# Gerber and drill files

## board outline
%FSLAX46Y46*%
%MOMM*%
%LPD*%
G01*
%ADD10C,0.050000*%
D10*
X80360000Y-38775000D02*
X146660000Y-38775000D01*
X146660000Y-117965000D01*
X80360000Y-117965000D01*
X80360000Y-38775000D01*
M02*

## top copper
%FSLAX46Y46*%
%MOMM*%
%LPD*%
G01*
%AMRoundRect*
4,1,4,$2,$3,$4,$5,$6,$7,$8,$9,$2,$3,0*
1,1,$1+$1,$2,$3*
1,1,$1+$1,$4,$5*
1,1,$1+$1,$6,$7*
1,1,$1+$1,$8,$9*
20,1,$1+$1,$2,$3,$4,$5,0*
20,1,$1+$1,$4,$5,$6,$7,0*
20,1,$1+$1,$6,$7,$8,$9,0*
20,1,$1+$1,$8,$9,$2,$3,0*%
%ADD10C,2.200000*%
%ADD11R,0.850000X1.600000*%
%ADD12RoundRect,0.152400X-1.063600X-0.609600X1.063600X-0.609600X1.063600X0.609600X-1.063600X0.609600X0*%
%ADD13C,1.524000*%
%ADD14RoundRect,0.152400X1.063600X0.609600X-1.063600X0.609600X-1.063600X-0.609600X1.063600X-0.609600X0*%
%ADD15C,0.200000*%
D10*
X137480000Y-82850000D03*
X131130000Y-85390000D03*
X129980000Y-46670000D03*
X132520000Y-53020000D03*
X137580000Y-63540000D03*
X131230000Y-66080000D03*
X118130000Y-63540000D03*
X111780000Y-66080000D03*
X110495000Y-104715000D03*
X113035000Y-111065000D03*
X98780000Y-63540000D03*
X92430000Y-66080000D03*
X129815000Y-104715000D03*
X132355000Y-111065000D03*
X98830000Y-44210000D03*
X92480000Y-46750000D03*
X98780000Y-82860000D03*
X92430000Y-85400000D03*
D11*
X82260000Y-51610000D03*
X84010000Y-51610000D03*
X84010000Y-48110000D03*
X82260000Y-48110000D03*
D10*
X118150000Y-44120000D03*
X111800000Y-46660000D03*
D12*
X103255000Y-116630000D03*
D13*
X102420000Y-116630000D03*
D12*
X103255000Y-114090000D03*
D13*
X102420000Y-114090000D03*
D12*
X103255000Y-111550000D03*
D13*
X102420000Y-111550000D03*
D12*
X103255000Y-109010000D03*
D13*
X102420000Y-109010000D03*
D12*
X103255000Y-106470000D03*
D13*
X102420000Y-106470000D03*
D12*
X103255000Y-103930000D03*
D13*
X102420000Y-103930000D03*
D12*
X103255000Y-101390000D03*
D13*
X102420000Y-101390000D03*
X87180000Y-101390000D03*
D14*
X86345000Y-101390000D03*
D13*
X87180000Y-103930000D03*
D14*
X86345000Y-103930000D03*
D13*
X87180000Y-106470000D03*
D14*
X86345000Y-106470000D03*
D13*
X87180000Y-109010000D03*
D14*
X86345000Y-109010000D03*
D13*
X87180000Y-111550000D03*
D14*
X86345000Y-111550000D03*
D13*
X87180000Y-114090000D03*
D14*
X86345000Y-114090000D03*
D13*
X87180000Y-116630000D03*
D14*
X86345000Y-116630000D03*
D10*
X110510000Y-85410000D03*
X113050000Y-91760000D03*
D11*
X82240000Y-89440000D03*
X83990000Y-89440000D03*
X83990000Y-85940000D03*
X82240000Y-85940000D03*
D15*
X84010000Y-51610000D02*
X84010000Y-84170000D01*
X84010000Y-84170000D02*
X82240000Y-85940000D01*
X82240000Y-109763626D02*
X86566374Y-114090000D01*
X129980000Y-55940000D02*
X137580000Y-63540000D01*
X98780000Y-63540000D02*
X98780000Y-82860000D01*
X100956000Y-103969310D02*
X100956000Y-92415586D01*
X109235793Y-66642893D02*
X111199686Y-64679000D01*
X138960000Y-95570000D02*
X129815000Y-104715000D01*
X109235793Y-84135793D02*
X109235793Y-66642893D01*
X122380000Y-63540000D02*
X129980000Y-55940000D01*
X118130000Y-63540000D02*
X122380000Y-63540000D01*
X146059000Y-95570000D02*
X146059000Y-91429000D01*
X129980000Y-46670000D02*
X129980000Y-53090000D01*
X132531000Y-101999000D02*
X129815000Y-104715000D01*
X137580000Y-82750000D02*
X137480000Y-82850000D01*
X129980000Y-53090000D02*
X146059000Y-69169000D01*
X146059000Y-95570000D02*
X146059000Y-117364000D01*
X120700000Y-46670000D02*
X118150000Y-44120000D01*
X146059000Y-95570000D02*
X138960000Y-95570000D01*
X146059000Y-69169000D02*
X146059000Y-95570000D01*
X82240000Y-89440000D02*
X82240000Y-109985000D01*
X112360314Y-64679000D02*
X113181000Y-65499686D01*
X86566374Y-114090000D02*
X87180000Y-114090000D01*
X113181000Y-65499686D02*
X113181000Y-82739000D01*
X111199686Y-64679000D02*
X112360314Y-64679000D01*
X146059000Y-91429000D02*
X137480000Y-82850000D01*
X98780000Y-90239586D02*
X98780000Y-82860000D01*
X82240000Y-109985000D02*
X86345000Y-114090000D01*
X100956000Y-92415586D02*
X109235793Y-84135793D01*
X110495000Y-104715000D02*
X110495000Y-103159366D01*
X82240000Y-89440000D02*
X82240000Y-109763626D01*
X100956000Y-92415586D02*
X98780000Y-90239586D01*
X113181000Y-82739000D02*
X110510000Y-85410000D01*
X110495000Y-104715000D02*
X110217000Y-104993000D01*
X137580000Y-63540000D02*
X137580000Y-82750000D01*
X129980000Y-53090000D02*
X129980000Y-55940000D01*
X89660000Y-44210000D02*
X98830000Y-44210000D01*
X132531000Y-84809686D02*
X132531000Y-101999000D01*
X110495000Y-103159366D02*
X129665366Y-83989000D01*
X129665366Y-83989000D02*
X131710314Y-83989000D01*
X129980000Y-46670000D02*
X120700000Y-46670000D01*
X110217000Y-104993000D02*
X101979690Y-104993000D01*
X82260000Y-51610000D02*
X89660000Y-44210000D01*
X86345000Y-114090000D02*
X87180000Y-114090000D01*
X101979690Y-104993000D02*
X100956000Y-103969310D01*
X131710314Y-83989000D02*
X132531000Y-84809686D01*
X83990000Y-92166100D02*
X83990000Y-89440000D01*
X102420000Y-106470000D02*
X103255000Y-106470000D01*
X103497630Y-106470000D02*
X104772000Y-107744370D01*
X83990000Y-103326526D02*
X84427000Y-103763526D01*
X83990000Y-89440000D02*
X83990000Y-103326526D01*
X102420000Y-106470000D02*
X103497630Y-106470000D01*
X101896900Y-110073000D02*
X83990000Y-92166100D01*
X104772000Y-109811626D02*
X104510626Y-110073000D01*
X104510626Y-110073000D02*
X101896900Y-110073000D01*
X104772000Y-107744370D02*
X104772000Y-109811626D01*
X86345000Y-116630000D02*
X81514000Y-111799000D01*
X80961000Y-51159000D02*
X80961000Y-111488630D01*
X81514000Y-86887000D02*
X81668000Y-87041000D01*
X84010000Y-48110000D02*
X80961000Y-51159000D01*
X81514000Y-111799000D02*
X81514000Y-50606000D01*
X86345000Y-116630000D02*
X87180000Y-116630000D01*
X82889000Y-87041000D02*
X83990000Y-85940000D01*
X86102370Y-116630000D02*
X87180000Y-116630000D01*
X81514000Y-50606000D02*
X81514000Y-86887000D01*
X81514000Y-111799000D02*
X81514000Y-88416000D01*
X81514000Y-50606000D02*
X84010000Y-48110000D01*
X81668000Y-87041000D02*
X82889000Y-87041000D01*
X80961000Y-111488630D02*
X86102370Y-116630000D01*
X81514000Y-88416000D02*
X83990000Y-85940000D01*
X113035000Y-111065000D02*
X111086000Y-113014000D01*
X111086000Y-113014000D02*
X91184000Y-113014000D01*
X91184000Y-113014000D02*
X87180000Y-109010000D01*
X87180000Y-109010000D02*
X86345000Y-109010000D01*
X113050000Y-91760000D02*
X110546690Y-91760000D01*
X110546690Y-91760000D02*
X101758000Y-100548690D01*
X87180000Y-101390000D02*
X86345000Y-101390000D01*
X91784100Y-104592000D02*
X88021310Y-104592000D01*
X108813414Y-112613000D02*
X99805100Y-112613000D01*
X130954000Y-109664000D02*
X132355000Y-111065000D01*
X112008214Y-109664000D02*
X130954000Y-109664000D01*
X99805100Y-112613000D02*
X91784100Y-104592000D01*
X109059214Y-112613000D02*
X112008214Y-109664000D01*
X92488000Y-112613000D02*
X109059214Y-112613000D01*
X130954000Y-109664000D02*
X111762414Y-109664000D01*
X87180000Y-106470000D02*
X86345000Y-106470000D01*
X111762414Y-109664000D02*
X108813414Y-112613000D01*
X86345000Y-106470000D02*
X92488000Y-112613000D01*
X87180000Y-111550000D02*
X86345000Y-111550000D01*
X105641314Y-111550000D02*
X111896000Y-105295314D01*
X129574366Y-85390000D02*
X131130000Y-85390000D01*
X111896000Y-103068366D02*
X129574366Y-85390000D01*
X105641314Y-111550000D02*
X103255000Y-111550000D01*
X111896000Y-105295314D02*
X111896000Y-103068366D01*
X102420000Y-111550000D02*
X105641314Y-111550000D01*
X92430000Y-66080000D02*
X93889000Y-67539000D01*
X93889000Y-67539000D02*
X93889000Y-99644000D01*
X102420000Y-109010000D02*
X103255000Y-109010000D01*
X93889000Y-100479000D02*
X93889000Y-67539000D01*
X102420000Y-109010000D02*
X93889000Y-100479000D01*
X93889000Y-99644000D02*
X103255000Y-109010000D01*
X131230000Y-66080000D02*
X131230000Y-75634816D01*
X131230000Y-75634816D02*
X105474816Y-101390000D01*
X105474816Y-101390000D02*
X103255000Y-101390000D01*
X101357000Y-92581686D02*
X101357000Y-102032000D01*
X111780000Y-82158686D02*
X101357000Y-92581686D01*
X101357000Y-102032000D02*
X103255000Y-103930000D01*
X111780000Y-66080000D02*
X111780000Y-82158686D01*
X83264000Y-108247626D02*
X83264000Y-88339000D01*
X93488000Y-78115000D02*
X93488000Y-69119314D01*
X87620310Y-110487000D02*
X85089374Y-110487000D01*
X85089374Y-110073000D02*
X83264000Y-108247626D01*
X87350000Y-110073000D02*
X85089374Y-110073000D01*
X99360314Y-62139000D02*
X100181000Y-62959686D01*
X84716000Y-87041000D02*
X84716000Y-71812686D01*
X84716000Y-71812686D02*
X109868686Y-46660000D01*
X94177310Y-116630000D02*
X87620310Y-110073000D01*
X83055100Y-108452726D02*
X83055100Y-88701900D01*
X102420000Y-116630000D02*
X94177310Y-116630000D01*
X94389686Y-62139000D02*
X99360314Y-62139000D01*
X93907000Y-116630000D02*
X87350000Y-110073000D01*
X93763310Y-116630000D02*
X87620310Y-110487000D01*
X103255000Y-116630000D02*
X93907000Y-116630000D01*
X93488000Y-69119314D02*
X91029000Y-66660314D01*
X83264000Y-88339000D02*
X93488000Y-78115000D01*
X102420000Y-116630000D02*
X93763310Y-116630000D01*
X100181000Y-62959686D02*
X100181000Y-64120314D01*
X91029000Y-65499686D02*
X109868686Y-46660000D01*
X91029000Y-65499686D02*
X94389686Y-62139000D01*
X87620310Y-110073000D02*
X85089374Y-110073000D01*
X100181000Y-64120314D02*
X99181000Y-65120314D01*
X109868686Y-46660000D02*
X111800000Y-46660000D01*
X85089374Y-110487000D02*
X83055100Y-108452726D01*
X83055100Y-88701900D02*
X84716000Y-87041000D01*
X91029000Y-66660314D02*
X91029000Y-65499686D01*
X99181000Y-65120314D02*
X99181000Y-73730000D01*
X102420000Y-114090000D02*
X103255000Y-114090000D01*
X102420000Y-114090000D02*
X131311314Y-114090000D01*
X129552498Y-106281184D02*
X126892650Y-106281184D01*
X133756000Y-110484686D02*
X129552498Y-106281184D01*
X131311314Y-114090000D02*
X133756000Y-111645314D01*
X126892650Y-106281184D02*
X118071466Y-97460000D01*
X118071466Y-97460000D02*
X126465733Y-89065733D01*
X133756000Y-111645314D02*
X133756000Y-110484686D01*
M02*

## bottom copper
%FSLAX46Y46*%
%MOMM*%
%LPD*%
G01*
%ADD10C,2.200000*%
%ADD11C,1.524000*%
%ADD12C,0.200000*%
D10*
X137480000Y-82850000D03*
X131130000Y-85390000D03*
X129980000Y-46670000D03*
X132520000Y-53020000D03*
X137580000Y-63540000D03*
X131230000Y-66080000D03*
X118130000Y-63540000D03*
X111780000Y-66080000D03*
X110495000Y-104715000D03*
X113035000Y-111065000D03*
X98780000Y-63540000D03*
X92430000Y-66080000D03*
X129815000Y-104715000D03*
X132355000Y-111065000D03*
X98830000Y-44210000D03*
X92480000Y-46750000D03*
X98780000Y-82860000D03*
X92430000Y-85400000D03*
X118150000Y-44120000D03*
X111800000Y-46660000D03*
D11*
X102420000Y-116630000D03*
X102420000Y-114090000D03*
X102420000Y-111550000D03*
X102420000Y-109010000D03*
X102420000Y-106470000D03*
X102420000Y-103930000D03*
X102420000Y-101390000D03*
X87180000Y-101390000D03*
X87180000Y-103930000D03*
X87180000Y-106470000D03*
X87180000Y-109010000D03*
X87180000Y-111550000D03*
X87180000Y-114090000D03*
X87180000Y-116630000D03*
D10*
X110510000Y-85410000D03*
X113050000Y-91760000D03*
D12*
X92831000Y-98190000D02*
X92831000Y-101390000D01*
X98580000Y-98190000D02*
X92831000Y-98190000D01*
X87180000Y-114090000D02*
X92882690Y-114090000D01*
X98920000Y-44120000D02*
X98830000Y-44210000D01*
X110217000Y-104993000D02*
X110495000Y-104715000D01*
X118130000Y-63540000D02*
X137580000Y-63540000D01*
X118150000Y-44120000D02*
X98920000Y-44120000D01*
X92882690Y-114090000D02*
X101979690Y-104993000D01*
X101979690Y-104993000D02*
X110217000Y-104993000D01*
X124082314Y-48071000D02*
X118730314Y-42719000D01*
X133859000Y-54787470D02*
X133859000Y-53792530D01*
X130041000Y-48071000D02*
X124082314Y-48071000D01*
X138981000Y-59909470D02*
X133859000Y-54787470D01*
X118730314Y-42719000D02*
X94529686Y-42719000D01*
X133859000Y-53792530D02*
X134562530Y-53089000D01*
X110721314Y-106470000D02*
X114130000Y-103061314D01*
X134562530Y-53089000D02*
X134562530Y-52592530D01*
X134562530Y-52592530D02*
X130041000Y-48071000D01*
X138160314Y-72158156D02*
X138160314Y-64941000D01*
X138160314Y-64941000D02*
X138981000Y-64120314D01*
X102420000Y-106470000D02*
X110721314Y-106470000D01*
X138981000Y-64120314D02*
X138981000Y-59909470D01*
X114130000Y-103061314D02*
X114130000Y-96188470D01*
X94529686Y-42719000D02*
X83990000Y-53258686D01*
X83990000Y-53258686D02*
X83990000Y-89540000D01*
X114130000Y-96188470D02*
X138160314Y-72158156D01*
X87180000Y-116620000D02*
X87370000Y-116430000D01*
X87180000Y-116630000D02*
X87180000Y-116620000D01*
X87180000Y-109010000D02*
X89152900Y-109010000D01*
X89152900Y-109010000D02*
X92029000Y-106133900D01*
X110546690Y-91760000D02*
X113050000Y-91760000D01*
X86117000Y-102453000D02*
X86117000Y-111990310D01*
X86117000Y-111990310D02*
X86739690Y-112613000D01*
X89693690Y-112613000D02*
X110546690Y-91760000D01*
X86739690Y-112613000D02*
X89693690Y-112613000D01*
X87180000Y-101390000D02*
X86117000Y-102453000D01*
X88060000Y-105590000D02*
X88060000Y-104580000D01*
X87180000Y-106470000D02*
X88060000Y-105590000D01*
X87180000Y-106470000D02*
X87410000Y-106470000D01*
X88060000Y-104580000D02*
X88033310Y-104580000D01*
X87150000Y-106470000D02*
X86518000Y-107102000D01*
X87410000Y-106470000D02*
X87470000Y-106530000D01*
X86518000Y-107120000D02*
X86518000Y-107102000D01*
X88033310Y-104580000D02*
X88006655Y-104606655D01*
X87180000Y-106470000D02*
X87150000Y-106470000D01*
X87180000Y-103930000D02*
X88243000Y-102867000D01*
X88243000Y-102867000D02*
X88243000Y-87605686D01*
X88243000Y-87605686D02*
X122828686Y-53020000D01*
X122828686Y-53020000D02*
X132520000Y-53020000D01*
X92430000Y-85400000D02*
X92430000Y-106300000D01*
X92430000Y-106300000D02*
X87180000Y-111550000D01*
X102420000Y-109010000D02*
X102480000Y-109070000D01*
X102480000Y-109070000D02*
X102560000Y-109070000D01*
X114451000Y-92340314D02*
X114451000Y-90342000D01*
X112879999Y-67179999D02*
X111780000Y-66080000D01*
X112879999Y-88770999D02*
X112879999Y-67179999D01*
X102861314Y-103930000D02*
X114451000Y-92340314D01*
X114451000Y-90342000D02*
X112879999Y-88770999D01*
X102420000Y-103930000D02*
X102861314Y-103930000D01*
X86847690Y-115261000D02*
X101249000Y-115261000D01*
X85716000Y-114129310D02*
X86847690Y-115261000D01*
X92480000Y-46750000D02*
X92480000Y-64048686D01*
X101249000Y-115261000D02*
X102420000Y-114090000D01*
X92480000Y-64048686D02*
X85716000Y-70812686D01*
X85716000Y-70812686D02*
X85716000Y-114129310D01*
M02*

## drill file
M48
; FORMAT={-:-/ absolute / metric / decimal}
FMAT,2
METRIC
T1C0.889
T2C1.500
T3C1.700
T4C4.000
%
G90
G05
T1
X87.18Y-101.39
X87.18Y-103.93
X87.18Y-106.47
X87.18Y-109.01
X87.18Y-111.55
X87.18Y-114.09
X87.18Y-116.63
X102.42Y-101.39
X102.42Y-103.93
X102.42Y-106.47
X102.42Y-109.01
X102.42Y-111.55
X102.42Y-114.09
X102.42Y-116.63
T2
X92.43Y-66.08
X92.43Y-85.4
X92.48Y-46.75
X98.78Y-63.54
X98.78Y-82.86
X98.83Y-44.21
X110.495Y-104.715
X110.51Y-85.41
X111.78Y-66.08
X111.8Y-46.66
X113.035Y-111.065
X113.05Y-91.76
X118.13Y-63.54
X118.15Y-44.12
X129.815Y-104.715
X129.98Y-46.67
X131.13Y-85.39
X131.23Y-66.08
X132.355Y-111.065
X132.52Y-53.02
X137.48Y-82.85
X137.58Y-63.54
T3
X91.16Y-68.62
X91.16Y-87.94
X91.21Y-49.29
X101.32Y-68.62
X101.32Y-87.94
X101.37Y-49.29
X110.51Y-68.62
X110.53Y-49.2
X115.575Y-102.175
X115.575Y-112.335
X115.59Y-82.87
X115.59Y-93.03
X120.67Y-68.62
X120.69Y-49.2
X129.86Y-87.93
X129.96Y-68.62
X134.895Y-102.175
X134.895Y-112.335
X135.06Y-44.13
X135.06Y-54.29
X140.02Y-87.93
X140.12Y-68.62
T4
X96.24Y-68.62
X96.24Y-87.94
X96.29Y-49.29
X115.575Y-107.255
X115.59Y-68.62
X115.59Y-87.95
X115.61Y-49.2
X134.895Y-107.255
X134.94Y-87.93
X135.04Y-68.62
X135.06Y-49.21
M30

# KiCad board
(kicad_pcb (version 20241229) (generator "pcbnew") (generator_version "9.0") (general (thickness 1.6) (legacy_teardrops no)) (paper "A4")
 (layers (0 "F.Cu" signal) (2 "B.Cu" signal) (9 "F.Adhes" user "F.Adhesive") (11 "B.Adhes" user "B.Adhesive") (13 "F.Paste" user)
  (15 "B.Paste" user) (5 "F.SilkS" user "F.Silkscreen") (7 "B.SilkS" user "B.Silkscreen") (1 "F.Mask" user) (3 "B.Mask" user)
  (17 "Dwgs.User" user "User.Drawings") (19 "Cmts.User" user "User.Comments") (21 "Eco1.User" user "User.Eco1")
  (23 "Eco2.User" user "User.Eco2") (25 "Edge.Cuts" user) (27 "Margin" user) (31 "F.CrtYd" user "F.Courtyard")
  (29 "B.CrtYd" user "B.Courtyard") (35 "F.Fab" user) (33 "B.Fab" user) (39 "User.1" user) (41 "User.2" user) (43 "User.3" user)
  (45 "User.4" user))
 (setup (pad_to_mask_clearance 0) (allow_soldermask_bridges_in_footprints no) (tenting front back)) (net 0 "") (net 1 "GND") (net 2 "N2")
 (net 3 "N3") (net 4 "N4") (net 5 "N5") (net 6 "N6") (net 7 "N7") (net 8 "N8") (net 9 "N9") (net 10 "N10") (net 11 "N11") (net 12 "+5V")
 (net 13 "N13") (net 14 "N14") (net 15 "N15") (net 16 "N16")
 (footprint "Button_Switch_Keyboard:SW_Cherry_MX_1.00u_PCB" (layer "F.Cu") (at 137.48 82.85)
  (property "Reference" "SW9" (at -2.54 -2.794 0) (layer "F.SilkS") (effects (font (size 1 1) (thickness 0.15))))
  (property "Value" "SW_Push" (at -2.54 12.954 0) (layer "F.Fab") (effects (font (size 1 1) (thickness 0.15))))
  (pad "" np_thru_hole circle (at -7.62 5.08) (size 1.7 1.7) (drill 1.7) (layers "*.Cu" "*.Mask"))
  (pad "" np_thru_hole circle (at -2.54 5.08) (size 4 4) (drill 4) (layers "*.Cu" "*.Mask"))
  (pad "" np_thru_hole circle (at 2.54 5.08) (size 1.7 1.7) (drill 1.7) (layers "*.Cu" "*.Mask"))
  (pad "1" thru_hole circle (at 0 0) (size 2.2 2.2) (drill 1.5) (layers "*.Cu" "*.Mask") (remove_unused_layers no) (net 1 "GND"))
  (pad "2" thru_hole circle (at -6.35 2.54) (size 2.2 2.2) (drill 1.5) (layers "*.Cu" "*.Mask") (remove_unused_layers no) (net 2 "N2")))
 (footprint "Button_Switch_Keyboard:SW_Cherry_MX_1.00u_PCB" (layer "F.Cu") (at 129.98 46.67 90)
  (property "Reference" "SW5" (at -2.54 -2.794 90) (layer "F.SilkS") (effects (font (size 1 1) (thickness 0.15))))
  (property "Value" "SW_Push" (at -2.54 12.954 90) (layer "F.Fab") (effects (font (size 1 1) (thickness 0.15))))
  (pad "" np_thru_hole circle (at -7.62 5.08 90) (size 1.7 1.7) (drill 1.7) (layers "*.Cu" "*.Mask"))
  (pad "" np_thru_hole circle (at -2.54 5.08 90) (size 4 4) (drill 4) (layers "*.Cu" "*.Mask"))
  (pad "" np_thru_hole circle (at 2.54 5.08 90) (size 1.7 1.7) (drill 1.7) (layers "*.Cu" "*.Mask"))
  (pad "1" thru_hole circle (at 0 0 90) (size 2.2 2.2) (drill 1.5) (layers "*.Cu" "*.Mask") (remove_unused_layers no) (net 1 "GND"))
  (pad "2" thru_hole circle (at -6.35 2.54 90) (size 2.2 2.2) (drill 1.5) (layers "*.Cu" "*.Mask") (remove_unused_layers no) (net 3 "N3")))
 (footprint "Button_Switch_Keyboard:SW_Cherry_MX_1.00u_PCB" (layer "F.Cu") (at 137.58 63.54)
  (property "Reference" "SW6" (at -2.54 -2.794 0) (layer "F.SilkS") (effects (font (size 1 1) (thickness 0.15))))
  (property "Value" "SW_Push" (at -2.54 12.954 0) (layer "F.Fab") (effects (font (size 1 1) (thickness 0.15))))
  (pad "" np_thru_hole circle (at -7.62 5.08) (size 1.7 1.7) (drill 1.7) (layers "*.Cu" "*.Mask"))
  (pad "" np_thru_hole circle (at -2.54 5.08) (size 4 4) (drill 4) (layers "*.Cu" "*.Mask"))
  (pad "" np_thru_hole circle (at 2.54 5.08) (size 1.7 1.7) (drill 1.7) (layers "*.Cu" "*.Mask"))
  (pad "1" thru_hole circle (at 0 0) (size 2.2 2.2) (drill 1.5) (layers "*.Cu" "*.Mask") (remove_unused_layers no) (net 1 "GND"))
  (pad "2" thru_hole circle (at -6.35 2.54) (size 2.2 2.2) (drill 1.5) (layers "*.Cu" "*.Mask") (remove_unused_layers no) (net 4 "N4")))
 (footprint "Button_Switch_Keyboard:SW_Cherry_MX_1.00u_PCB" (layer "F.Cu") (at 118.13 63.54)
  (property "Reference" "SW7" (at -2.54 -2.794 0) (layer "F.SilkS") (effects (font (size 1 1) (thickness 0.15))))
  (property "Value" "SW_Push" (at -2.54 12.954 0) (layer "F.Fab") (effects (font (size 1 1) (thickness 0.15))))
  (pad "" np_thru_hole circle (at -7.62 5.08) (size 1.7 1.7) (drill 1.7) (layers "*.Cu" "*.Mask"))
  (pad "" np_thru_hole circle (at -2.54 5.08) (size 4 4) (drill 4) (layers "*.Cu" "*.Mask"))
  (pad "" np_thru_hole circle (at 2.54 5.08) (size 1.7 1.7) (drill 1.7) (layers "*.Cu" "*.Mask"))
  (pad "1" thru_hole circle (at 0 0) (size 2.2 2.2) (drill 1.5) (layers "*.Cu" "*.Mask") (remove_unused_layers no) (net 1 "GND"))
  (pad "2" thru_hole circle (at -6.35 2.54) (size 2.2 2.2) (drill 1.5) (layers "*.Cu" "*.Mask") (remove_unused_layers no) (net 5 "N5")))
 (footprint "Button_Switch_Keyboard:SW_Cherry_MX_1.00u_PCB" (layer "F.Cu") (at 110.495 104.715 90)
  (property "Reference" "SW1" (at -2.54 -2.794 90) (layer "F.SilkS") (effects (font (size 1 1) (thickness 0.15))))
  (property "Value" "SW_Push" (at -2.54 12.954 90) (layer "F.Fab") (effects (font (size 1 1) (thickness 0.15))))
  (pad "" np_thru_hole circle (at -7.62 5.08 90) (size 1.7 1.7) (drill 1.7) (layers "*.Cu" "*.Mask"))
  (pad "" np_thru_hole circle (at -2.54 5.08 90) (size 4 4) (drill 4) (layers "*.Cu" "*.Mask"))
  (pad "" np_thru_hole circle (at 2.54 5.08 90) (size 1.7 1.7) (drill 1.7) (layers "*.Cu" "*.Mask"))
  (pad "1" thru_hole circle (at 0 0 90) (size 2.2 2.2) (drill 1.5) (layers "*.Cu" "*.Mask") (remove_unused_layers no) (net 1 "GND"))
  (pad "2" thru_hole circle (at -6.35 2.54 90) (size 2.2 2.2) (drill 1.5) (layers "*.Cu" "*.Mask") (remove_unused_layers no) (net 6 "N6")))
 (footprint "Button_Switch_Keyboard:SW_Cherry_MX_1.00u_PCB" (layer "F.Cu") (at 98.78 63.54)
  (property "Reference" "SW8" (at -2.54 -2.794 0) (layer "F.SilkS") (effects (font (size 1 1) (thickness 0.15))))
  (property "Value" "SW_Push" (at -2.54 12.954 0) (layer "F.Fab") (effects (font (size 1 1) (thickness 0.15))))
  (pad "" np_thru_hole circle (at -7.62 5.08) (size 1.7 1.7) (drill 1.7) (layers "*.Cu" "*.Mask"))
  (pad "" np_thru_hole circle (at -2.54 5.08) (size 4 4) (drill 4) (layers "*.Cu" "*.Mask"))
  (pad "" np_thru_hole circle (at 2.54 5.08) (size 1.7 1.7) (drill 1.7) (layers "*.Cu" "*.Mask"))
  (pad "1" thru_hole circle (at 0 0) (size 2.2 2.2) (drill 1.5) (layers "*.Cu" "*.Mask") (remove_unused_layers no) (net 1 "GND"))
  (pad "2" thru_hole circle (at -6.35 2.54) (size 2.2 2.2) (drill 1.5) (layers "*.Cu" "*.Mask") (remove_unused_layers no) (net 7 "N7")))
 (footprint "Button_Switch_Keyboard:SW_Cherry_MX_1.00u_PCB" (layer "F.Cu") (at 129.815 104.715 90)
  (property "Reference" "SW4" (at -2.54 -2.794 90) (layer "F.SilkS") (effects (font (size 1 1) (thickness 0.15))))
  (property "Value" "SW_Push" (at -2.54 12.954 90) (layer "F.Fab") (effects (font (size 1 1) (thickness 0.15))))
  (pad "" np_thru_hole circle (at -7.62 5.08 90) (size 1.7 1.7) (drill 1.7) (layers "*.Cu" "*.Mask"))
  (pad "" np_thru_hole circle (at -2.54 5.08 90) (size 4 4) (drill 4) (layers "*.Cu" "*.Mask"))
  (pad "" np_thru_hole circle (at 2.54 5.08 90) (size 1.7 1.7) (drill 1.7) (layers "*.Cu" "*.Mask"))
  (pad "1" thru_hole circle (at 0 0 90) (size 2.2 2.2) (drill 1.5) (layers "*.Cu" "*.Mask") (remove_unused_layers no) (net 1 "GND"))
  (pad "2" thru_hole circle (at -6.35 2.54 90) (size 2.2 2.2) (drill 1.5) (layers "*.Cu" "*.Mask") (remove_unused_layers no) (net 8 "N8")))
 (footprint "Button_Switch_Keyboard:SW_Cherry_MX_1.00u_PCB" (layer "F.Cu") (at 98.83 44.21)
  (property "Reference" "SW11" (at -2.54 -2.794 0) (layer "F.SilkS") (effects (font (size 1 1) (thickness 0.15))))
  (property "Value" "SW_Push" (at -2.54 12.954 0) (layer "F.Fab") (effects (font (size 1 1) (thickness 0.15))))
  (pad "" np_thru_hole circle (at -7.62 5.08) (size 1.7 1.7) (drill 1.7) (layers "*.Cu" "*.Mask"))
  (pad "" np_thru_hole circle (at -2.54 5.08) (size 4 4) (drill 4) (layers "*.Cu" "*.Mask"))
  (pad "" np_thru_hole circle (at 2.54 5.08) (size 1.7 1.7) (drill 1.7) (layers "*.Cu" "*.Mask"))
  (pad "1" thru_hole circle (at 0 0) (size 2.2 2.2) (drill 1.5) (layers "*.Cu" "*.Mask") (remove_unused_layers no) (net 1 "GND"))
  (pad "2" thru_hole circle (at -6.35 2.54) (size 2.2 2.2) (drill 1.5) (layers "*.Cu" "*.Mask") (remove_unused_layers no) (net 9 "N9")))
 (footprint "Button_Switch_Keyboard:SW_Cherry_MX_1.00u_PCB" (layer "F.Cu") (at 98.78 82.86)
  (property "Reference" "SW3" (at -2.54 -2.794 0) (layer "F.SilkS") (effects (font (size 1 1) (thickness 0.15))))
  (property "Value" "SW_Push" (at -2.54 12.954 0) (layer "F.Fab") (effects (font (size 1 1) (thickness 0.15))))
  (pad "" np_thru_hole circle (at -7.62 5.08) (size 1.7 1.7) (drill 1.7) (layers "*.Cu" "*.Mask"))
  (pad "" np_thru_hole circle (at -2.54 5.08) (size 4 4) (drill 4) (layers "*.Cu" "*.Mask"))
  (pad "" np_thru_hole circle (at 2.54 5.08) (size 1.7 1.7) (drill 1.7) (layers "*.Cu" "*.Mask"))
  (pad "1" thru_hole circle (at 0 0) (size 2.2 2.2) (drill 1.5) (layers "*.Cu" "*.Mask") (remove_unused_layers no) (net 1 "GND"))
  (pad "2" thru_hole circle (at -6.35 2.54) (size 2.2 2.2) (drill 1.5) (layers "*.Cu" "*.Mask") (remove_unused_layers no) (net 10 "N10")))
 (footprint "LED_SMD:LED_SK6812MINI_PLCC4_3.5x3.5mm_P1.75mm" (layer "F.Cu") (at 83.135 49.86 90)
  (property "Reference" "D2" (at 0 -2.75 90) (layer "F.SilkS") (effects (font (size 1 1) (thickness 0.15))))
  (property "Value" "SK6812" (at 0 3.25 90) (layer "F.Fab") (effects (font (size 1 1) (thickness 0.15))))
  (pad "1" smd rect (at -1.75 -0.875 90) (size 1.6 0.85) (layers "F.Cu" "F.Mask" "F.Paste") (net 1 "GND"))
  (pad "2" smd rect (at -1.75 0.875 90) (size 1.6 0.85) (layers "F.Cu" "F.Mask" "F.Paste") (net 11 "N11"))
  (pad "3" smd rect (at 1.75 0.875 90) (size 1.6 0.85) (layers "F.Cu" "F.Mask" "F.Paste") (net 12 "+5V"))
  (pad "4" smd rect (at 1.75 -0.875 90) (size 1.6 0.85) (layers "F.Cu" "F.Mask" "F.Paste") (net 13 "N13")))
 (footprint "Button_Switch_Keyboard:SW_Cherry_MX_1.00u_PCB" (layer "F.Cu") (at 118.15 44.12)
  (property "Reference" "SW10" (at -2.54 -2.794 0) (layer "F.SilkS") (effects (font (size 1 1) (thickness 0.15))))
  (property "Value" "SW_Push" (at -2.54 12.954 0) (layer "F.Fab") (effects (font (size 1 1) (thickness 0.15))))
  (pad "" np_thru_hole circle (at -7.62 5.08) (size 1.7 1.7) (drill 1.7) (layers "*.Cu" "*.Mask"))
  (pad "" np_thru_hole circle (at -2.54 5.08) (size 4 4) (drill 4) (layers "*.Cu" "*.Mask"))
  (pad "" np_thru_hole circle (at 2.54 5.08) (size 1.7 1.7) (drill 1.7) (layers "*.Cu" "*.Mask"))
  (pad "1" thru_hole circle (at 0 0) (size 2.2 2.2) (drill 1.5) (layers "*.Cu" "*.Mask") (remove_unused_layers no) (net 1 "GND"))
  (pad "2" thru_hole circle (at -6.35 2.54) (size 2.2 2.2) (drill 1.5) (layers "*.Cu" "*.Mask") (remove_unused_layers no) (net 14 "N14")))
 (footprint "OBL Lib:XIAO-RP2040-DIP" (layer "F.Cu") (at 94.8 109.01 180)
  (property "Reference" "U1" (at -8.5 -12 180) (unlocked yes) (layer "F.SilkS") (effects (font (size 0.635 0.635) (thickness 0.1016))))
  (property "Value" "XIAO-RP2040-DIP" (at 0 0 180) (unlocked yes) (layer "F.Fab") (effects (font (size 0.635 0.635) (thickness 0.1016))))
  (pad "1" smd roundrect (at -8.455 -7.62) (size 2.432 1.524) (layers "F.Cu" "F.Mask") (roundrect_rratio 0.1) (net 14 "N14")
   (thermal_bridge_angle 45))
  (pad "1" thru_hole circle (at -7.62 -7.62) (size 1.524 1.524) (drill 0.889) (layers "*.Cu" "*.Mask") (remove_unused_layers no)
   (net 14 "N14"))
  (pad "2" smd roundrect (at -8.455 -5.08) (size 2.432 1.524) (layers "F.Cu" "F.Mask") (roundrect_rratio 0.1) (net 9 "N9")
   (thermal_bridge_angle 45))
  (pad "2" thru_hole circle (at -7.62 -5.08) (size 1.524 1.524) (drill 0.889) (layers "*.Cu" "*.Mask") (remove_unused_layers no)
   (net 9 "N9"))
  (pad "3" smd roundrect (at -8.455 -2.54) (size 2.432 1.524) (layers "F.Cu" "F.Mask") (roundrect_rratio 0.1) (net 2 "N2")
   (thermal_bridge_angle 45))
  (pad "3" thru_hole circle (at -7.62 -2.54) (size 1.524 1.524) (drill 0.889) (layers "*.Cu" "*.Mask") (remove_unused_layers no)
   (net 2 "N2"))
  (pad "4" smd roundrect (at -8.455 0) (size 2.432 1.524) (layers "F.Cu" "F.Mask") (roundrect_rratio 0.1) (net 7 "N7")
   (thermal_bridge_angle 45))
  (pad "4" thru_hole circle (at -7.62 0) (size 1.524 1.524) (drill 0.889) (layers "*.Cu" "*.Mask") (remove_unused_layers no) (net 7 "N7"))
  (pad "5" smd roundrect (at -8.455 2.54) (size 2.432 1.524) (layers "F.Cu" "F.Mask") (roundrect_rratio 0.1) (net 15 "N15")
   (thermal_bridge_angle 45))
  (pad "5" thru_hole circle (at -7.62 2.54) (size 1.524 1.524) (drill 0.889) (layers "*.Cu" "*.Mask") (remove_unused_layers no)
   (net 15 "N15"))
  (pad "6" smd roundrect (at -8.455 5.08) (size 2.432 1.524) (layers "F.Cu" "F.Mask") (roundrect_rratio 0.1) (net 5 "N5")
   (thermal_bridge_angle 45))
  (pad "6" thru_hole circle (at -7.62 5.08) (size 1.524 1.524) (drill 0.889) (layers "*.Cu" "*.Mask") (remove_unused_layers no) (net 5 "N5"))
  (pad "7" smd roundrect (at -8.455 7.62) (size 2.432 1.524) (layers "F.Cu" "F.Mask") (roundrect_rratio 0.1) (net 4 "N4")
   (thermal_bridge_angle 45))
  (pad "7" thru_hole circle (at -7.62 7.62) (size 1.524 1.524) (drill 0.889) (layers "*.Cu" "*.Mask") (remove_unused_layers no) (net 4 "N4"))
  (pad "8" thru_hole circle (at 7.62 7.62 180) (size 1.524 1.524) (drill 0.889) (layers "*.Cu" "*.Mask") (remove_unused_layers no)
   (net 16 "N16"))
  (pad "8" smd roundrect (at 8.455 7.62 180) (size 2.432 1.524) (layers "F.Cu" "F.Mask") (roundrect_rratio 0.1) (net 16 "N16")
   (thermal_bridge_angle 45))
  (pad "9" thru_hole circle (at 7.62 5.08 180) (size 1.524 1.524) (drill 0.889) (layers "*.Cu" "*.Mask") (remove_unused_layers no)
   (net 3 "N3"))
  (pad "9" smd roundrect (at 8.455 5.08 180) (size 2.432 1.524) (layers "F.Cu" "F.Mask") (roundrect_rratio 0.1) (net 3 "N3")
   (thermal_bridge_angle 45))
  (pad "10" thru_hole circle (at 7.62 2.54 180) (size 1.524 1.524) (drill 0.889) (layers "*.Cu" "*.Mask") (remove_unused_layers no)
   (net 8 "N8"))
  (pad "10" smd roundrect (at 8.455 2.54 180) (size 2.432 1.524) (layers "F.Cu" "F.Mask") (roundrect_rratio 0.1) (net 8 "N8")
   (thermal_bridge_angle 45))
  (pad "11" thru_hole circle (at 7.62 0 180) (size 1.524 1.524) (drill 0.889) (layers "*.Cu" "*.Mask") (remove_unused_layers no)
   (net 6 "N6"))
  (pad "11" smd roundrect (at 8.455 0 180) (size 2.432 1.524) (layers "F.Cu" "F.Mask") (roundrect_rratio 0.1) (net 6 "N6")
   (thermal_bridge_angle 45))
  (pad "12" thru_hole circle (at 7.62 -2.54 180) (size 1.524 1.524) (drill 0.889) (layers "*.Cu" "*.Mask") (remove_unused_layers no)
   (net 10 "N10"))
  (pad "12" smd roundrect (at 8.455 -2.54 180) (size 2.432 1.524) (layers "F.Cu" "F.Mask") (roundrect_rratio 0.1) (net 10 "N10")
   (thermal_bridge_angle 45))
  (pad "13" thru_hole circle (at 7.62 -5.08 180) (size 1.524 1.524) (drill 0.889) (layers "*.Cu" "*.Mask") (remove_unused_layers no)
   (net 1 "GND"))
  (pad "13" smd roundrect (at 8.455 -5.08 180) (size 2.432 1.524) (layers "F.Cu" "F.Mask") (roundrect_rratio 0.1) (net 1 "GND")
   (thermal_bridge_angle 45))
  (pad "14" thru_hole circle (at 7.62 -7.62 180) (size 1.524 1.524) (drill 0.889) (layers "*.Cu" "*.Mask") (remove_unused_layers no)
   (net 12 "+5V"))
  (pad "14" smd roundrect (at 8.455 -7.62 180) (size 2.432 1.524) (layers "F.Cu" "F.Mask") (roundrect_rratio 0.1) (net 12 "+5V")
   (thermal_bridge_angle 45)))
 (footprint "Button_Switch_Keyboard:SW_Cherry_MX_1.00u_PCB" (layer "F.Cu") (at 110.51 85.41 90)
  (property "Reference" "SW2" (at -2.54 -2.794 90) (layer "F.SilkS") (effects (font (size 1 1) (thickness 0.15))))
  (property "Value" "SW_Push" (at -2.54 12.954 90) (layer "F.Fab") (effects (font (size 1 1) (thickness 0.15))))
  (pad "" np_thru_hole circle (at -7.62 5.08 90) (size 1.7 1.7) (drill 1.7) (layers "*.Cu" "*.Mask"))
  (pad "" np_thru_hole circle (at -2.54 5.08 90) (size 4 4) (drill 4) (layers "*.Cu" "*.Mask"))
  (pad "" np_thru_hole circle (at 2.54 5.08 90) (size 1.7 1.7) (drill 1.7) (layers "*.Cu" "*.Mask"))
  (pad "1" thru_hole circle (at 0 0 90) (size 2.2 2.2) (drill 1.5) (layers "*.Cu" "*.Mask") (remove_unused_layers no) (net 1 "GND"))
  (pad "2" thru_hole circle (at -6.35 2.54 90) (size 2.2 2.2) (drill 1.5) (layers "*.Cu" "*.Mask") (remove_unused_layers no) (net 16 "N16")))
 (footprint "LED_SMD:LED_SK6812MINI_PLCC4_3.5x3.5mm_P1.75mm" (layer "F.Cu") (at 83.115 87.69 90)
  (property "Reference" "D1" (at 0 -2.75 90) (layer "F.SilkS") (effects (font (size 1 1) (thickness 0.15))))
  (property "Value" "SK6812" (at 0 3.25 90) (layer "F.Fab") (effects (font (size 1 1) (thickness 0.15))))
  (pad "1" smd rect (at -1.75 -0.875 90) (size 1.6 0.85) (layers "F.Cu" "F.Mask" "F.Paste") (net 1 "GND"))
  (pad "2" smd rect (at -1.75 0.875 90) (size 1.6 0.85) (layers "F.Cu" "F.Mask" "F.Paste") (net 15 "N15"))
  (pad "3" smd rect (at 1.75 0.875 90) (size 1.6 0.85) (layers "F.Cu" "F.Mask" "F.Paste") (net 12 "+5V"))
  (pad "4" smd rect (at 1.75 -0.875 90) (size 1.6 0.85) (layers "F.Cu" "F.Mask" "F.Paste") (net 11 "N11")))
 (gr_rect (start 80.36 38.775) (end 146.66 117.965) (stroke (width 0.05) (type default)) (fill no) (layer "Edge.Cuts"))
 (segment (start 92.831 98.19) (end 92.831 101.39) (width 0.2) (layer "B.Cu") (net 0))
 (segment (start 98.58 98.19) (end 92.831 98.19) (width 0.2) (layer "B.Cu") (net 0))
 (segment (start 84.01 51.61) (end 84.01 84.17) (width 0.2) (layer "F.Cu") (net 11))
 (segment (start 84.01 84.17) (end 82.24 85.94) (width 0.2) (layer "F.Cu") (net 11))
 (segment (start 82.24 109.763626) (end 86.566374 114.09) (width 0.2) (layer "F.Cu") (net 1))
 (segment (start 129.98 55.94) (end 137.58 63.54) (width 0.2) (layer "F.Cu") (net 1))
 (segment (start 98.78 63.54) (end 98.78 82.86) (width 0.2) (layer "F.Cu") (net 1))
 (segment (start 100.956 103.96931) (end 100.956 92.415586) (width 0.2) (layer "F.Cu") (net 1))
 (segment (start 109.235793 66.642893) (end 111.199686 64.679) (width 0.2) (layer "F.Cu") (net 1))
 (segment (start 138.96 95.57) (end 129.815 104.715) (width 0.2) (layer "F.Cu") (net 1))
 (segment (start 109.235793 84.135793) (end 109.235793 66.642893) (width 0.2) (layer "F.Cu") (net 1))
 (segment (start 122.38 63.54) (end 129.98 55.94) (width 0.2) (layer "F.Cu") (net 1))
 (segment (start 118.13 63.54) (end 122.38 63.54) (width 0.2) (layer "F.Cu") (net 1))
 (segment (start 146.059 95.57) (end 146.059 91.429) (width 0.2) (layer "F.Cu") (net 1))
 (segment (start 129.98 46.67) (end 129.98 53.09) (width 0.2) (layer "F.Cu") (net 1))
 (segment (start 132.531 101.999) (end 129.815 104.715) (width 0.2) (layer "F.Cu") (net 1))
 (segment (start 137.58 82.75) (end 137.48 82.85) (width 0.2) (layer "F.Cu") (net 1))
 (segment (start 129.98 53.09) (end 146.059 69.169) (width 0.2) (layer "F.Cu") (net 1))
 (segment (start 146.059 95.57) (end 146.059 117.364) (width 0.2) (layer "F.Cu") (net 1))
 (segment (start 120.7 46.67) (end 118.15 44.12) (width 0.2) (layer "F.Cu") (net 1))
 (segment (start 146.059 95.57) (end 138.96 95.57) (width 0.2) (layer "F.Cu") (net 1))
 (segment (start 146.059 69.169) (end 146.059 95.57) (width 0.2) (layer "F.Cu") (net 1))
 (segment (start 82.24 89.44) (end 82.24 109.985) (width 0.2) (layer "F.Cu") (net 1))
 (segment (start 112.360314 64.679) (end 113.181 65.499686) (width 0.2) (layer "F.Cu") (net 1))
 (segment (start 86.566374 114.09) (end 87.18 114.09) (width 0.2) (layer "F.Cu") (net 1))
 (segment (start 113.181 65.499686) (end 113.181 82.739) (width 0.2) (layer "F.Cu") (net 1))
 (segment (start 111.199686 64.679) (end 112.360314 64.679) (width 0.2) (layer "F.Cu") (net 1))
 (segment (start 146.059 91.429) (end 137.48 82.85) (width 0.2) (layer "F.Cu") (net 1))
 (segment (start 98.78 90.239586) (end 98.78 82.86) (width 0.2) (layer "F.Cu") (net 1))
 (segment (start 82.24 109.985) (end 86.345 114.09) (width 0.2) (layer "F.Cu") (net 1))
 (segment (start 100.956 92.415586) (end 109.235793 84.135793) (width 0.2) (layer "F.Cu") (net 1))
 (segment (start 110.495 104.715) (end 110.495 103.159366) (width 0.2) (layer "F.Cu") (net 1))
 (segment (start 82.24 89.44) (end 82.24 109.763626) (width 0.2) (layer "F.Cu") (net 1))
 (segment (start 100.956 92.415586) (end 98.78 90.239586) (width 0.2) (layer "F.Cu") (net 1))
 (segment (start 113.181 82.739) (end 110.51 85.41) (width 0.2) (layer "F.Cu") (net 1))
 (segment (start 110.495 104.715) (end 110.217 104.993) (width 0.2) (layer "F.Cu") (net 1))
 (segment (start 137.58 63.54) (end 137.58 82.75) (width 0.2) (layer "F.Cu") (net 1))
 (segment (start 129.98 53.09) (end 129.98 55.94) (width 0.2) (layer "F.Cu") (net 1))
 (segment (start 89.66 44.21) (end 98.83 44.21) (width 0.2) (layer "F.Cu") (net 1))
 (segment (start 132.531 84.809686) (end 132.531 101.999) (width 0.2) (layer "F.Cu") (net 1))
 (segment (start 110.495 103.159366) (end 129.665366 83.989) (width 0.2) (layer "F.Cu") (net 1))
 (segment (start 129.665366 83.989) (end 131.710314 83.989) (width 0.2) (layer "F.Cu") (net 1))
 (segment (start 129.98 46.67) (end 120.7 46.67) (width 0.2) (layer "F.Cu") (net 1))
 (segment (start 110.217 104.993) (end 101.97969 104.993) (width 0.2) (layer "F.Cu") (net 1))
 (segment (start 82.26 51.61) (end 89.66 44.21) (width 0.2) (layer "F.Cu") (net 1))
 (segment (start 86.345 114.09) (end 87.18 114.09) (width 0.2) (layer "F.Cu") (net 1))
 (segment (start 101.97969 104.993) (end 100.956 103.96931) (width 0.2) (layer "F.Cu") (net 1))
 (segment (start 131.710314 83.989) (end 132.531 84.809686) (width 0.2) (layer "F.Cu") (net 1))
 (segment (start 87.18 114.09) (end 92.88269 114.09) (width 0.2) (layer "B.Cu") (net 1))
 (segment (start 98.92 44.12) (end 98.83 44.21) (width 0.2) (layer "B.Cu") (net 1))
 (segment (start 110.217 104.993) (end 110.495 104.715) (width 0.2) (layer "B.Cu") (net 1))
 (segment (start 118.13 63.54) (end 137.58 63.54) (width 0.2) (layer "B.Cu") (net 1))
 (segment (start 118.15 44.12) (end 98.92 44.12) (width 0.2) (layer "B.Cu") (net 1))
 (segment (start 92.88269 114.09) (end 101.97969 104.993) (width 0.2) (layer "B.Cu") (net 1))
 (segment (start 101.97969 104.993) (end 110.217 104.993) (width 0.2) (layer "B.Cu") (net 1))
 (segment (start 83.99 92.1661) (end 83.99 89.44) (width 0.2) (layer "F.Cu") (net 15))
 (segment (start 102.42 106.47) (end 103.255 106.47) (width 0.2) (layer "F.Cu") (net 15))
 (segment (start 103.49763 106.47) (end 104.772 107.74437) (width 0.2) (layer "F.Cu") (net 15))
 (segment (start 83.99 103.326526) (end 84.427 103.763526) (width 0.2) (layer "F.Cu") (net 15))
 (segment (start 83.99 89.44) (end 83.99 103.326526) (width 0.2) (layer "F.Cu") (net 15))
 (segment (start 102.42 106.47) (end 103.49763 106.47) (width 0.2) (layer "F.Cu") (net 15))
 (segment (start 101.8969 110.073) (end 83.99 92.1661) (width 0.2) (layer "F.Cu") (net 15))
 (segment (start 104.772 109.811626) (end 104.510626 110.073) (width 0.2) (layer "F.Cu") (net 15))
 (segment (start 104.510626 110.073) (end 101.8969 110.073) (width 0.2) (layer "F.Cu") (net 15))
 (segment (start 104.772 107.74437) (end 104.772 109.811626) (width 0.2) (layer "F.Cu") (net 15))
 (segment (start 124.082314 48.071) (end 118.730314 42.719) (width 0.2) (layer "B.Cu") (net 15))
 (segment (start 133.859 54.78747) (end 133.859 53.79253) (width 0.2) (layer "B.Cu") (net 15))
 (segment (start 130.041 48.071) (end 124.082314 48.071) (width 0.2) (layer "B.Cu") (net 15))
 (segment (start 138.981 59.90947) (end 133.859 54.78747) (width 0.2) (layer "B.Cu") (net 15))
 (segment (start 118.730314 42.719) (end 94.529686 42.719) (width 0.2) (layer "B.Cu") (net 15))
 (segment (start 133.859 53.79253) (end 134.56253 53.089) (width 0.2) (layer "B.Cu") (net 15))
 (segment (start 110.721314 106.47) (end 114.13 103.061314) (width 0.2) (layer "B.Cu") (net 15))
 (segment (start 134.56253 53.089) (end 134.56253 52.59253) (width 0.2) (layer "B.Cu") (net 15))
 (segment (start 134.56253 52.59253) (end 130.041 48.071) (width 0.2) (layer "B.Cu") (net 15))
 (segment (start 138.160314 72.158156) (end 138.160314 64.941) (width 0.2) (layer "B.Cu") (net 15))
 (segment (start 138.160314 64.941) (end 138.981 64.120314) (width 0.2) (layer "B.Cu") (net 15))
 (segment (start 102.42 106.47) (end 110.721314 106.47) (width 0.2) (layer "B.Cu") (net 15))
 (segment (start 138.981 64.120314) (end 138.981 59.90947) (width 0.2) (layer "B.Cu") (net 15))
 (segment (start 114.13 103.061314) (end 114.13 96.18847) (width 0.2) (layer "B.Cu") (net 15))
 (segment (start 94.529686 42.719) (end 83.99 53.258686) (width 0.2) (layer "B.Cu") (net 15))
 (segment (start 83.99 53.258686) (end 83.99 89.54) (width 0.2) (layer "B.Cu") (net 15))
 (segment (start 114.13 96.18847) (end 138.160314 72.158156) (width 0.2) (layer "B.Cu") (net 15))
 (segment (start 86.345 116.63) (end 81.514 111.799) (width 0.2) (layer "F.Cu") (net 12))
 (segment (start 80.961 51.159) (end 80.961 111.48863) (width 0.2) (layer "F.Cu") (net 12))
 (segment (start 81.514 86.887) (end 81.668 87.041) (width 0.2) (layer "F.Cu") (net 12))
 (segment (start 84.01 48.11) (end 80.961 51.159) (width 0.2) (layer "F.Cu") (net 12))
 (segment (start 81.514 111.799) (end 81.514 50.606) (width 0.2) (layer "F.Cu") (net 12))
 (segment (start 86.345 116.63) (end 87.18 116.63) (width 0.2) (layer "F.Cu") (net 12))
 (segment (start 82.889 87.041) (end 83.99 85.94) (width 0.2) (layer "F.Cu") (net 12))
 (segment (start 86.10237 116.63) (end 87.18 116.63) (width 0.2) (layer "F.Cu") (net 12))
 (segment (start 81.514 50.606) (end 81.514 86.887) (width 0.2) (layer "F.Cu") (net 12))
 (segment (start 81.514 111.799) (end 81.514 88.416) (width 0.2) (layer "F.Cu") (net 12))
 (segment (start 81.514 50.606) (end 84.01 48.11) (width 0.2) (layer "F.Cu") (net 12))
 (segment (start 81.668 87.041) (end 82.889 87.041) (width 0.2) (layer "F.Cu") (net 12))
 (segment (start 80.961 111.48863) (end 86.10237 116.63) (width 0.2) (layer "F.Cu") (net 12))
 (segment (start 81.514 88.416) (end 83.99 85.94) (width 0.2) (layer "F.Cu") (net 12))
 (segment (start 87.18 116.62) (end 87.37 116.43) (width 0.2) (layer "B.Cu") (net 12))
 (segment (start 87.18 116.63) (end 87.18 116.62) (width 0.2) (layer "B.Cu") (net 12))
 (segment (start 113.035 111.065) (end 111.086 113.014) (width 0.2) (layer "F.Cu") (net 6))
 (segment (start 111.086 113.014) (end 91.184 113.014) (width 0.2) (layer "F.Cu") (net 6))
 (segment (start 91.184 113.014) (end 87.18 109.01) (width 0.2) (layer "F.Cu") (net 6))
 (segment (start 87.18 109.01) (end 86.345 109.01) (width 0.2) (layer "F.Cu") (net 6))
 (segment (start 87.18 109.01) (end 89.1529 109.01) (width 0.2) (layer "B.Cu") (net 6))
 (segment (start 89.1529 109.01) (end 92.029 106.1339) (width 0.2) (layer "B.Cu") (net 6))
 (segment (start 113.05 91.76) (end 110.54669 91.76) (width 0.2) (layer "F.Cu") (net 16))
 (segment (start 110.54669 91.76) (end 101.758 100.54869) (width 0.2) (layer "F.Cu") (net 16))
 (segment (start 87.18 101.39) (end 86.345 101.39) (width 0.2) (layer "F.Cu") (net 16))
 (segment (start 110.54669 91.76) (end 113.05 91.76) (width 0.2) (layer "B.Cu") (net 16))
 (segment (start 86.117 102.453) (end 86.117 111.99031) (width 0.2) (layer "B.Cu") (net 16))
 (segment (start 86.117 111.99031) (end 86.73969 112.613) (width 0.2) (layer "B.Cu") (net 16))
 (segment (start 89.69369 112.613) (end 110.54669 91.76) (width 0.2) (layer "B.Cu") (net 16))
 (segment (start 86.73969 112.613) (end 89.69369 112.613) (width 0.2) (layer "B.Cu") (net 16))
 (segment (start 87.18 101.39) (end 86.117 102.453) (width 0.2) (layer "B.Cu") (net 16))
 (segment (start 91.7841 104.592) (end 88.02131 104.592) (width 0.2) (layer "F.Cu") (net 8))
 (segment (start 108.813414 112.613) (end 99.8051 112.613) (width 0.2) (layer "F.Cu") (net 8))
 (segment (start 130.954 109.664) (end 132.355 111.065) (width 0.2) (layer "F.Cu") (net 8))
 (segment (start 112.008214 109.664) (end 130.954 109.664) (width 0.2) (layer "F.Cu") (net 8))
 (segment (start 99.8051 112.613) (end 91.7841 104.592) (width 0.2) (layer "F.Cu") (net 8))
 (segment (start 109.059214 112.613) (end 112.008214 109.664) (width 0.2) (layer "F.Cu") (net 8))
 (segment (start 92.488 112.613) (end 109.059214 112.613) (width 0.2) (layer "F.Cu") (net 8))
 (segment (start 130.954 109.664) (end 111.762414 109.664) (width 0.2) (layer "F.Cu") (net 8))
 (segment (start 87.18 106.47) (end 86.345 106.47) (width 0.2) (layer "F.Cu") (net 8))
 (segment (start 111.762414 109.664) (end 108.813414 112.613) (width 0.2) (layer "F.Cu") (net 8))
 (segment (start 86.345 106.47) (end 92.488 112.613) (width 0.2) (layer "F.Cu") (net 8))
 (segment (start 88.06 105.59) (end 88.06 104.58) (width 0.2) (layer "B.Cu") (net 8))
 (segment (start 87.18 106.47) (end 88.06 105.59) (width 0.2) (layer "B.Cu") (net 8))
 (segment (start 87.18 106.47) (end 87.41 106.47) (width 0.2) (layer "B.Cu") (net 8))
 (segment (start 88.06 104.58) (end 88.03331 104.58) (width 0.2) (layer "B.Cu") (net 8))
 (segment (start 87.15 106.47) (end 86.518 107.102) (width 0.2) (layer "B.Cu") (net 8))
 (segment (start 87.41 106.47) (end 87.47 106.53) (width 0.2) (layer "B.Cu") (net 8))
 (segment (start 86.518 107.12) (end 86.518 107.102) (width 0.2) (layer "B.Cu") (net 8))
 (segment (start 88.03331 104.58) (end 88.006655 104.606655) (width 0.2) (layer "B.Cu") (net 8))
 (segment (start 87.18 106.47) (end 87.15 106.47) (width 0.2) (layer "B.Cu") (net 8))
 (segment (start 87.18 103.93) (end 88.243 102.867) (width 0.2) (layer "B.Cu") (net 3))
 (segment (start 88.243 102.867) (end 88.243 87.605686) (width 0.2) (layer "B.Cu") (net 3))
 (segment (start 88.243 87.605686) (end 122.828686 53.02) (width 0.2) (layer "B.Cu") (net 3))
 (segment (start 122.828686 53.02) (end 132.52 53.02) (width 0.2) (layer "B.Cu") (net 3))
 (segment (start 87.18 111.55) (end 86.345 111.55) (width 0.2) (layer "F.Cu") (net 10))
 (segment (start 92.43 85.4) (end 92.43 106.3) (width 0.2) (layer "B.Cu") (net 10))
 (segment (start 92.43 106.3) (end 87.18 111.55) (width 0.2) (layer "B.Cu") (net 10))
 (segment (start 105.641314 111.55) (end 111.896 105.295314) (width 0.2) (layer "F.Cu") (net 2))
 (segment (start 129.574366 85.39) (end 131.13 85.39) (width 0.2) (layer "F.Cu") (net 2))
 (segment (start 111.896 103.068366) (end 129.574366 85.39) (width 0.2) (layer "F.Cu") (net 2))
 (segment (start 105.641314 111.55) (end 103.255 111.55) (width 0.2) (layer "F.Cu") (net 2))
 (segment (start 111.896 105.295314) (end 111.896 103.068366) (width 0.2) (layer "F.Cu") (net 2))
 (segment (start 102.42 111.55) (end 105.641314 111.55) (width 0.2) (layer "F.Cu") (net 2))
 (segment (start 92.43 66.08) (end 93.889 67.539) (width 0.2) (layer "F.Cu") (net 7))
 (segment (start 93.889 67.539) (end 93.889 99.644) (width 0.2) (layer "F.Cu") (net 7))
 (segment (start 102.42 109.01) (end 103.255 109.01) (width 0.2) (layer "F.Cu") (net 7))
 (segment (start 93.889 100.479) (end 93.889 67.539) (width 0.2) (layer "F.Cu") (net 7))
 (segment (start 102.42 109.01) (end 93.889 100.479) (width 0.2) (layer "F.Cu") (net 7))
 (segment (start 93.889 99.644) (end 103.255 109.01) (width 0.2) (layer "F.Cu") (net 7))
 (segment (start 102.42 109.01) (end 102.48 109.07) (width 0.2) (layer "B.Cu") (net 7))
 (segment (start 102.48 109.07) (end 102.56 109.07) (width 0.2) (layer "B.Cu") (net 7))
 (segment (start 131.23 66.08) (end 131.23 75.634816) (width 0.2) (layer "F.Cu") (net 4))
 (segment (start 131.23 75.634816) (end 105.474816 101.39) (width 0.2) (layer "F.Cu") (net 4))
 (segment (start 105.474816 101.39) (end 103.255 101.39) (width 0.2) (layer "F.Cu") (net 4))
 (segment (start 101.357 92.581686) (end 101.357 102.032) (width 0.2) (layer "F.Cu") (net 5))
 (segment (start 111.78 82.158686) (end 101.357 92.581686) (width 0.2) (layer "F.Cu") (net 5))
 (segment (start 101.357 102.032) (end 103.255 103.93) (width 0.2) (layer "F.Cu") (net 5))
 (segment (start 111.78 66.08) (end 111.78 82.158686) (width 0.2) (layer "F.Cu") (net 5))
 (segment (start 114.451 92.340314) (end 114.451 90.342) (width 0.2) (layer "B.Cu") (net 5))
 (segment (start 112.879999 67.179999) (end 111.78 66.08) (width 0.2) (layer "B.Cu") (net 5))
 (segment (start 112.879999 88.770999) (end 112.879999 67.179999) (width 0.2) (layer "B.Cu") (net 5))
 (segment (start 102.861314 103.93) (end 114.451 92.340314) (width 0.2) (layer "B.Cu") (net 5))
 (segment (start 114.451 90.342) (end 112.879999 88.770999) (width 0.2) (layer "B.Cu") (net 5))
 (segment (start 102.42 103.93) (end 102.861314 103.93) (width 0.2) (layer "B.Cu") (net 5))
 (segment (start 83.264 108.247626) (end 83.264 88.339) (width 0.2) (layer "F.Cu") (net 14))
 (segment (start 93.488 78.115) (end 93.488 69.119314) (width 0.2) (layer "F.Cu") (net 14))
 (segment (start 87.62031 110.487) (end 85.089374 110.487) (width 0.2) (layer "F.Cu") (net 14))
 (segment (start 85.089374 110.073) (end 83.264 108.247626) (width 0.2) (layer "F.Cu") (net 14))
 (segment (start 87.35 110.073) (end 85.089374 110.073) (width 0.2) (layer "F.Cu") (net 14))
 (segment (start 99.360314 62.139) (end 100.181 62.959686) (width 0.2) (layer "F.Cu") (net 14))
 (segment (start 84.716 87.041) (end 84.716 71.812686) (width 0.2) (layer "F.Cu") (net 14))
 (segment (start 84.716 71.812686) (end 109.868686 46.66) (width 0.2) (layer "F.Cu") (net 14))
 (segment (start 94.17731 116.63) (end 87.62031 110.073) (width 0.2) (layer "F.Cu") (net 14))
 (segment (start 83.0551 108.452726) (end 83.0551 88.7019) (width 0.2) (layer "F.Cu") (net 14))
 (segment (start 102.42 116.63) (end 94.17731 116.63) (width 0.2) (layer "F.Cu") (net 14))
 (segment (start 94.389686 62.139) (end 99.360314 62.139) (width 0.2) (layer "F.Cu") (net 14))
 (segment (start 93.907 116.63) (end 87.35 110.073) (width 0.2) (layer "F.Cu") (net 14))
 (segment (start 93.76331 116.63) (end 87.62031 110.487) (width 0.2) (layer "F.Cu") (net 14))
 (segment (start 103.255 116.63) (end 93.907 116.63) (width 0.2) (layer "F.Cu") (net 14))
 (segment (start 93.488 69.119314) (end 91.029 66.660314) (width 0.2) (layer "F.Cu") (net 14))
 (segment (start 83.264 88.339) (end 93.488 78.115) (width 0.2) (layer "F.Cu") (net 14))
 (segment (start 102.42 116.63) (end 93.76331 116.63) (width 0.2) (layer "F.Cu") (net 14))
 (segment (start 100.181 62.959686) (end 100.181 64.120314) (width 0.2) (layer "F.Cu") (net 14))
 (segment (start 91.029 65.499686) (end 109.868686 46.66) (width 0.2) (layer "F.Cu") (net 14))
 (segment (start 91.029 65.499686) (end 94.389686 62.139) (width 0.2) (layer "F.Cu") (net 14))
 (segment (start 87.62031 110.073) (end 85.089374 110.073) (width 0.2) (layer "F.Cu") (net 14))
 (segment (start 100.181 64.120314) (end 99.181 65.120314) (width 0.2) (layer "F.Cu") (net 14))
 (segment (start 109.868686 46.66) (end 111.8 46.66) (width 0.2) (layer "F.Cu") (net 14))
 (segment (start 85.089374 110.487) (end 83.0551 108.452726) (width 0.2) (layer "F.Cu") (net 14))
 (segment (start 83.0551 88.7019) (end 84.716 87.041) (width 0.2) (layer "F.Cu") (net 14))
 (segment (start 91.029 66.660314) (end 91.029 65.499686) (width 0.2) (layer "F.Cu") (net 14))
 (segment (start 99.181 65.120314) (end 99.181 73.73) (width 0.2) (layer "F.Cu") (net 14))
 (segment (start 102.42 114.09) (end 103.255 114.09) (width 0.2) (layer "F.Cu") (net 9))
 (segment (start 102.42 114.09) (end 131.311314 114.09) (width 0.2) (layer "F.Cu") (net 9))
 (segment (start 129.552498 106.281184) (end 126.89265 106.281184) (width 0.2) (layer "F.Cu") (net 9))
 (segment (start 133.756 110.484686) (end 129.552498 106.281184) (width 0.2) (layer "F.Cu") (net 9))
 (segment (start 131.311314 114.09) (end 133.756 111.645314) (width 0.2) (layer "F.Cu") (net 9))
 (segment (start 126.89265 106.281184) (end 118.071466 97.46) (width 0.2) (layer "F.Cu") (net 9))
 (segment (start 118.071466 97.46) (end 126.465733 89.065733) (width 0.2) (layer "F.Cu") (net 9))
 (segment (start 133.756 111.645314) (end 133.756 110.484686) (width 0.2) (layer "F.Cu") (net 9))
 (segment (start 86.84769 115.261) (end 101.249 115.261) (width 0.2) (layer "B.Cu") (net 9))
 (segment (start 85.716 114.12931) (end 86.84769 115.261) (width 0.2) (layer "B.Cu") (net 9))
 (segment (start 92.48 46.75) (end 92.48 64.048686) (width 0.2) (layer "B.Cu") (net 9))
 (segment (start 101.249 115.261) (end 102.42 114.09) (width 0.2) (layer "B.Cu") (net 9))
 (segment (start 92.48 64.048686) (end 85.716 70.812686) (width 0.2) (layer "B.Cu") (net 9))
 (segment (start 85.716 70.812686) (end 85.716 114.12931) (width 0.2) (layer "B.Cu") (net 9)))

